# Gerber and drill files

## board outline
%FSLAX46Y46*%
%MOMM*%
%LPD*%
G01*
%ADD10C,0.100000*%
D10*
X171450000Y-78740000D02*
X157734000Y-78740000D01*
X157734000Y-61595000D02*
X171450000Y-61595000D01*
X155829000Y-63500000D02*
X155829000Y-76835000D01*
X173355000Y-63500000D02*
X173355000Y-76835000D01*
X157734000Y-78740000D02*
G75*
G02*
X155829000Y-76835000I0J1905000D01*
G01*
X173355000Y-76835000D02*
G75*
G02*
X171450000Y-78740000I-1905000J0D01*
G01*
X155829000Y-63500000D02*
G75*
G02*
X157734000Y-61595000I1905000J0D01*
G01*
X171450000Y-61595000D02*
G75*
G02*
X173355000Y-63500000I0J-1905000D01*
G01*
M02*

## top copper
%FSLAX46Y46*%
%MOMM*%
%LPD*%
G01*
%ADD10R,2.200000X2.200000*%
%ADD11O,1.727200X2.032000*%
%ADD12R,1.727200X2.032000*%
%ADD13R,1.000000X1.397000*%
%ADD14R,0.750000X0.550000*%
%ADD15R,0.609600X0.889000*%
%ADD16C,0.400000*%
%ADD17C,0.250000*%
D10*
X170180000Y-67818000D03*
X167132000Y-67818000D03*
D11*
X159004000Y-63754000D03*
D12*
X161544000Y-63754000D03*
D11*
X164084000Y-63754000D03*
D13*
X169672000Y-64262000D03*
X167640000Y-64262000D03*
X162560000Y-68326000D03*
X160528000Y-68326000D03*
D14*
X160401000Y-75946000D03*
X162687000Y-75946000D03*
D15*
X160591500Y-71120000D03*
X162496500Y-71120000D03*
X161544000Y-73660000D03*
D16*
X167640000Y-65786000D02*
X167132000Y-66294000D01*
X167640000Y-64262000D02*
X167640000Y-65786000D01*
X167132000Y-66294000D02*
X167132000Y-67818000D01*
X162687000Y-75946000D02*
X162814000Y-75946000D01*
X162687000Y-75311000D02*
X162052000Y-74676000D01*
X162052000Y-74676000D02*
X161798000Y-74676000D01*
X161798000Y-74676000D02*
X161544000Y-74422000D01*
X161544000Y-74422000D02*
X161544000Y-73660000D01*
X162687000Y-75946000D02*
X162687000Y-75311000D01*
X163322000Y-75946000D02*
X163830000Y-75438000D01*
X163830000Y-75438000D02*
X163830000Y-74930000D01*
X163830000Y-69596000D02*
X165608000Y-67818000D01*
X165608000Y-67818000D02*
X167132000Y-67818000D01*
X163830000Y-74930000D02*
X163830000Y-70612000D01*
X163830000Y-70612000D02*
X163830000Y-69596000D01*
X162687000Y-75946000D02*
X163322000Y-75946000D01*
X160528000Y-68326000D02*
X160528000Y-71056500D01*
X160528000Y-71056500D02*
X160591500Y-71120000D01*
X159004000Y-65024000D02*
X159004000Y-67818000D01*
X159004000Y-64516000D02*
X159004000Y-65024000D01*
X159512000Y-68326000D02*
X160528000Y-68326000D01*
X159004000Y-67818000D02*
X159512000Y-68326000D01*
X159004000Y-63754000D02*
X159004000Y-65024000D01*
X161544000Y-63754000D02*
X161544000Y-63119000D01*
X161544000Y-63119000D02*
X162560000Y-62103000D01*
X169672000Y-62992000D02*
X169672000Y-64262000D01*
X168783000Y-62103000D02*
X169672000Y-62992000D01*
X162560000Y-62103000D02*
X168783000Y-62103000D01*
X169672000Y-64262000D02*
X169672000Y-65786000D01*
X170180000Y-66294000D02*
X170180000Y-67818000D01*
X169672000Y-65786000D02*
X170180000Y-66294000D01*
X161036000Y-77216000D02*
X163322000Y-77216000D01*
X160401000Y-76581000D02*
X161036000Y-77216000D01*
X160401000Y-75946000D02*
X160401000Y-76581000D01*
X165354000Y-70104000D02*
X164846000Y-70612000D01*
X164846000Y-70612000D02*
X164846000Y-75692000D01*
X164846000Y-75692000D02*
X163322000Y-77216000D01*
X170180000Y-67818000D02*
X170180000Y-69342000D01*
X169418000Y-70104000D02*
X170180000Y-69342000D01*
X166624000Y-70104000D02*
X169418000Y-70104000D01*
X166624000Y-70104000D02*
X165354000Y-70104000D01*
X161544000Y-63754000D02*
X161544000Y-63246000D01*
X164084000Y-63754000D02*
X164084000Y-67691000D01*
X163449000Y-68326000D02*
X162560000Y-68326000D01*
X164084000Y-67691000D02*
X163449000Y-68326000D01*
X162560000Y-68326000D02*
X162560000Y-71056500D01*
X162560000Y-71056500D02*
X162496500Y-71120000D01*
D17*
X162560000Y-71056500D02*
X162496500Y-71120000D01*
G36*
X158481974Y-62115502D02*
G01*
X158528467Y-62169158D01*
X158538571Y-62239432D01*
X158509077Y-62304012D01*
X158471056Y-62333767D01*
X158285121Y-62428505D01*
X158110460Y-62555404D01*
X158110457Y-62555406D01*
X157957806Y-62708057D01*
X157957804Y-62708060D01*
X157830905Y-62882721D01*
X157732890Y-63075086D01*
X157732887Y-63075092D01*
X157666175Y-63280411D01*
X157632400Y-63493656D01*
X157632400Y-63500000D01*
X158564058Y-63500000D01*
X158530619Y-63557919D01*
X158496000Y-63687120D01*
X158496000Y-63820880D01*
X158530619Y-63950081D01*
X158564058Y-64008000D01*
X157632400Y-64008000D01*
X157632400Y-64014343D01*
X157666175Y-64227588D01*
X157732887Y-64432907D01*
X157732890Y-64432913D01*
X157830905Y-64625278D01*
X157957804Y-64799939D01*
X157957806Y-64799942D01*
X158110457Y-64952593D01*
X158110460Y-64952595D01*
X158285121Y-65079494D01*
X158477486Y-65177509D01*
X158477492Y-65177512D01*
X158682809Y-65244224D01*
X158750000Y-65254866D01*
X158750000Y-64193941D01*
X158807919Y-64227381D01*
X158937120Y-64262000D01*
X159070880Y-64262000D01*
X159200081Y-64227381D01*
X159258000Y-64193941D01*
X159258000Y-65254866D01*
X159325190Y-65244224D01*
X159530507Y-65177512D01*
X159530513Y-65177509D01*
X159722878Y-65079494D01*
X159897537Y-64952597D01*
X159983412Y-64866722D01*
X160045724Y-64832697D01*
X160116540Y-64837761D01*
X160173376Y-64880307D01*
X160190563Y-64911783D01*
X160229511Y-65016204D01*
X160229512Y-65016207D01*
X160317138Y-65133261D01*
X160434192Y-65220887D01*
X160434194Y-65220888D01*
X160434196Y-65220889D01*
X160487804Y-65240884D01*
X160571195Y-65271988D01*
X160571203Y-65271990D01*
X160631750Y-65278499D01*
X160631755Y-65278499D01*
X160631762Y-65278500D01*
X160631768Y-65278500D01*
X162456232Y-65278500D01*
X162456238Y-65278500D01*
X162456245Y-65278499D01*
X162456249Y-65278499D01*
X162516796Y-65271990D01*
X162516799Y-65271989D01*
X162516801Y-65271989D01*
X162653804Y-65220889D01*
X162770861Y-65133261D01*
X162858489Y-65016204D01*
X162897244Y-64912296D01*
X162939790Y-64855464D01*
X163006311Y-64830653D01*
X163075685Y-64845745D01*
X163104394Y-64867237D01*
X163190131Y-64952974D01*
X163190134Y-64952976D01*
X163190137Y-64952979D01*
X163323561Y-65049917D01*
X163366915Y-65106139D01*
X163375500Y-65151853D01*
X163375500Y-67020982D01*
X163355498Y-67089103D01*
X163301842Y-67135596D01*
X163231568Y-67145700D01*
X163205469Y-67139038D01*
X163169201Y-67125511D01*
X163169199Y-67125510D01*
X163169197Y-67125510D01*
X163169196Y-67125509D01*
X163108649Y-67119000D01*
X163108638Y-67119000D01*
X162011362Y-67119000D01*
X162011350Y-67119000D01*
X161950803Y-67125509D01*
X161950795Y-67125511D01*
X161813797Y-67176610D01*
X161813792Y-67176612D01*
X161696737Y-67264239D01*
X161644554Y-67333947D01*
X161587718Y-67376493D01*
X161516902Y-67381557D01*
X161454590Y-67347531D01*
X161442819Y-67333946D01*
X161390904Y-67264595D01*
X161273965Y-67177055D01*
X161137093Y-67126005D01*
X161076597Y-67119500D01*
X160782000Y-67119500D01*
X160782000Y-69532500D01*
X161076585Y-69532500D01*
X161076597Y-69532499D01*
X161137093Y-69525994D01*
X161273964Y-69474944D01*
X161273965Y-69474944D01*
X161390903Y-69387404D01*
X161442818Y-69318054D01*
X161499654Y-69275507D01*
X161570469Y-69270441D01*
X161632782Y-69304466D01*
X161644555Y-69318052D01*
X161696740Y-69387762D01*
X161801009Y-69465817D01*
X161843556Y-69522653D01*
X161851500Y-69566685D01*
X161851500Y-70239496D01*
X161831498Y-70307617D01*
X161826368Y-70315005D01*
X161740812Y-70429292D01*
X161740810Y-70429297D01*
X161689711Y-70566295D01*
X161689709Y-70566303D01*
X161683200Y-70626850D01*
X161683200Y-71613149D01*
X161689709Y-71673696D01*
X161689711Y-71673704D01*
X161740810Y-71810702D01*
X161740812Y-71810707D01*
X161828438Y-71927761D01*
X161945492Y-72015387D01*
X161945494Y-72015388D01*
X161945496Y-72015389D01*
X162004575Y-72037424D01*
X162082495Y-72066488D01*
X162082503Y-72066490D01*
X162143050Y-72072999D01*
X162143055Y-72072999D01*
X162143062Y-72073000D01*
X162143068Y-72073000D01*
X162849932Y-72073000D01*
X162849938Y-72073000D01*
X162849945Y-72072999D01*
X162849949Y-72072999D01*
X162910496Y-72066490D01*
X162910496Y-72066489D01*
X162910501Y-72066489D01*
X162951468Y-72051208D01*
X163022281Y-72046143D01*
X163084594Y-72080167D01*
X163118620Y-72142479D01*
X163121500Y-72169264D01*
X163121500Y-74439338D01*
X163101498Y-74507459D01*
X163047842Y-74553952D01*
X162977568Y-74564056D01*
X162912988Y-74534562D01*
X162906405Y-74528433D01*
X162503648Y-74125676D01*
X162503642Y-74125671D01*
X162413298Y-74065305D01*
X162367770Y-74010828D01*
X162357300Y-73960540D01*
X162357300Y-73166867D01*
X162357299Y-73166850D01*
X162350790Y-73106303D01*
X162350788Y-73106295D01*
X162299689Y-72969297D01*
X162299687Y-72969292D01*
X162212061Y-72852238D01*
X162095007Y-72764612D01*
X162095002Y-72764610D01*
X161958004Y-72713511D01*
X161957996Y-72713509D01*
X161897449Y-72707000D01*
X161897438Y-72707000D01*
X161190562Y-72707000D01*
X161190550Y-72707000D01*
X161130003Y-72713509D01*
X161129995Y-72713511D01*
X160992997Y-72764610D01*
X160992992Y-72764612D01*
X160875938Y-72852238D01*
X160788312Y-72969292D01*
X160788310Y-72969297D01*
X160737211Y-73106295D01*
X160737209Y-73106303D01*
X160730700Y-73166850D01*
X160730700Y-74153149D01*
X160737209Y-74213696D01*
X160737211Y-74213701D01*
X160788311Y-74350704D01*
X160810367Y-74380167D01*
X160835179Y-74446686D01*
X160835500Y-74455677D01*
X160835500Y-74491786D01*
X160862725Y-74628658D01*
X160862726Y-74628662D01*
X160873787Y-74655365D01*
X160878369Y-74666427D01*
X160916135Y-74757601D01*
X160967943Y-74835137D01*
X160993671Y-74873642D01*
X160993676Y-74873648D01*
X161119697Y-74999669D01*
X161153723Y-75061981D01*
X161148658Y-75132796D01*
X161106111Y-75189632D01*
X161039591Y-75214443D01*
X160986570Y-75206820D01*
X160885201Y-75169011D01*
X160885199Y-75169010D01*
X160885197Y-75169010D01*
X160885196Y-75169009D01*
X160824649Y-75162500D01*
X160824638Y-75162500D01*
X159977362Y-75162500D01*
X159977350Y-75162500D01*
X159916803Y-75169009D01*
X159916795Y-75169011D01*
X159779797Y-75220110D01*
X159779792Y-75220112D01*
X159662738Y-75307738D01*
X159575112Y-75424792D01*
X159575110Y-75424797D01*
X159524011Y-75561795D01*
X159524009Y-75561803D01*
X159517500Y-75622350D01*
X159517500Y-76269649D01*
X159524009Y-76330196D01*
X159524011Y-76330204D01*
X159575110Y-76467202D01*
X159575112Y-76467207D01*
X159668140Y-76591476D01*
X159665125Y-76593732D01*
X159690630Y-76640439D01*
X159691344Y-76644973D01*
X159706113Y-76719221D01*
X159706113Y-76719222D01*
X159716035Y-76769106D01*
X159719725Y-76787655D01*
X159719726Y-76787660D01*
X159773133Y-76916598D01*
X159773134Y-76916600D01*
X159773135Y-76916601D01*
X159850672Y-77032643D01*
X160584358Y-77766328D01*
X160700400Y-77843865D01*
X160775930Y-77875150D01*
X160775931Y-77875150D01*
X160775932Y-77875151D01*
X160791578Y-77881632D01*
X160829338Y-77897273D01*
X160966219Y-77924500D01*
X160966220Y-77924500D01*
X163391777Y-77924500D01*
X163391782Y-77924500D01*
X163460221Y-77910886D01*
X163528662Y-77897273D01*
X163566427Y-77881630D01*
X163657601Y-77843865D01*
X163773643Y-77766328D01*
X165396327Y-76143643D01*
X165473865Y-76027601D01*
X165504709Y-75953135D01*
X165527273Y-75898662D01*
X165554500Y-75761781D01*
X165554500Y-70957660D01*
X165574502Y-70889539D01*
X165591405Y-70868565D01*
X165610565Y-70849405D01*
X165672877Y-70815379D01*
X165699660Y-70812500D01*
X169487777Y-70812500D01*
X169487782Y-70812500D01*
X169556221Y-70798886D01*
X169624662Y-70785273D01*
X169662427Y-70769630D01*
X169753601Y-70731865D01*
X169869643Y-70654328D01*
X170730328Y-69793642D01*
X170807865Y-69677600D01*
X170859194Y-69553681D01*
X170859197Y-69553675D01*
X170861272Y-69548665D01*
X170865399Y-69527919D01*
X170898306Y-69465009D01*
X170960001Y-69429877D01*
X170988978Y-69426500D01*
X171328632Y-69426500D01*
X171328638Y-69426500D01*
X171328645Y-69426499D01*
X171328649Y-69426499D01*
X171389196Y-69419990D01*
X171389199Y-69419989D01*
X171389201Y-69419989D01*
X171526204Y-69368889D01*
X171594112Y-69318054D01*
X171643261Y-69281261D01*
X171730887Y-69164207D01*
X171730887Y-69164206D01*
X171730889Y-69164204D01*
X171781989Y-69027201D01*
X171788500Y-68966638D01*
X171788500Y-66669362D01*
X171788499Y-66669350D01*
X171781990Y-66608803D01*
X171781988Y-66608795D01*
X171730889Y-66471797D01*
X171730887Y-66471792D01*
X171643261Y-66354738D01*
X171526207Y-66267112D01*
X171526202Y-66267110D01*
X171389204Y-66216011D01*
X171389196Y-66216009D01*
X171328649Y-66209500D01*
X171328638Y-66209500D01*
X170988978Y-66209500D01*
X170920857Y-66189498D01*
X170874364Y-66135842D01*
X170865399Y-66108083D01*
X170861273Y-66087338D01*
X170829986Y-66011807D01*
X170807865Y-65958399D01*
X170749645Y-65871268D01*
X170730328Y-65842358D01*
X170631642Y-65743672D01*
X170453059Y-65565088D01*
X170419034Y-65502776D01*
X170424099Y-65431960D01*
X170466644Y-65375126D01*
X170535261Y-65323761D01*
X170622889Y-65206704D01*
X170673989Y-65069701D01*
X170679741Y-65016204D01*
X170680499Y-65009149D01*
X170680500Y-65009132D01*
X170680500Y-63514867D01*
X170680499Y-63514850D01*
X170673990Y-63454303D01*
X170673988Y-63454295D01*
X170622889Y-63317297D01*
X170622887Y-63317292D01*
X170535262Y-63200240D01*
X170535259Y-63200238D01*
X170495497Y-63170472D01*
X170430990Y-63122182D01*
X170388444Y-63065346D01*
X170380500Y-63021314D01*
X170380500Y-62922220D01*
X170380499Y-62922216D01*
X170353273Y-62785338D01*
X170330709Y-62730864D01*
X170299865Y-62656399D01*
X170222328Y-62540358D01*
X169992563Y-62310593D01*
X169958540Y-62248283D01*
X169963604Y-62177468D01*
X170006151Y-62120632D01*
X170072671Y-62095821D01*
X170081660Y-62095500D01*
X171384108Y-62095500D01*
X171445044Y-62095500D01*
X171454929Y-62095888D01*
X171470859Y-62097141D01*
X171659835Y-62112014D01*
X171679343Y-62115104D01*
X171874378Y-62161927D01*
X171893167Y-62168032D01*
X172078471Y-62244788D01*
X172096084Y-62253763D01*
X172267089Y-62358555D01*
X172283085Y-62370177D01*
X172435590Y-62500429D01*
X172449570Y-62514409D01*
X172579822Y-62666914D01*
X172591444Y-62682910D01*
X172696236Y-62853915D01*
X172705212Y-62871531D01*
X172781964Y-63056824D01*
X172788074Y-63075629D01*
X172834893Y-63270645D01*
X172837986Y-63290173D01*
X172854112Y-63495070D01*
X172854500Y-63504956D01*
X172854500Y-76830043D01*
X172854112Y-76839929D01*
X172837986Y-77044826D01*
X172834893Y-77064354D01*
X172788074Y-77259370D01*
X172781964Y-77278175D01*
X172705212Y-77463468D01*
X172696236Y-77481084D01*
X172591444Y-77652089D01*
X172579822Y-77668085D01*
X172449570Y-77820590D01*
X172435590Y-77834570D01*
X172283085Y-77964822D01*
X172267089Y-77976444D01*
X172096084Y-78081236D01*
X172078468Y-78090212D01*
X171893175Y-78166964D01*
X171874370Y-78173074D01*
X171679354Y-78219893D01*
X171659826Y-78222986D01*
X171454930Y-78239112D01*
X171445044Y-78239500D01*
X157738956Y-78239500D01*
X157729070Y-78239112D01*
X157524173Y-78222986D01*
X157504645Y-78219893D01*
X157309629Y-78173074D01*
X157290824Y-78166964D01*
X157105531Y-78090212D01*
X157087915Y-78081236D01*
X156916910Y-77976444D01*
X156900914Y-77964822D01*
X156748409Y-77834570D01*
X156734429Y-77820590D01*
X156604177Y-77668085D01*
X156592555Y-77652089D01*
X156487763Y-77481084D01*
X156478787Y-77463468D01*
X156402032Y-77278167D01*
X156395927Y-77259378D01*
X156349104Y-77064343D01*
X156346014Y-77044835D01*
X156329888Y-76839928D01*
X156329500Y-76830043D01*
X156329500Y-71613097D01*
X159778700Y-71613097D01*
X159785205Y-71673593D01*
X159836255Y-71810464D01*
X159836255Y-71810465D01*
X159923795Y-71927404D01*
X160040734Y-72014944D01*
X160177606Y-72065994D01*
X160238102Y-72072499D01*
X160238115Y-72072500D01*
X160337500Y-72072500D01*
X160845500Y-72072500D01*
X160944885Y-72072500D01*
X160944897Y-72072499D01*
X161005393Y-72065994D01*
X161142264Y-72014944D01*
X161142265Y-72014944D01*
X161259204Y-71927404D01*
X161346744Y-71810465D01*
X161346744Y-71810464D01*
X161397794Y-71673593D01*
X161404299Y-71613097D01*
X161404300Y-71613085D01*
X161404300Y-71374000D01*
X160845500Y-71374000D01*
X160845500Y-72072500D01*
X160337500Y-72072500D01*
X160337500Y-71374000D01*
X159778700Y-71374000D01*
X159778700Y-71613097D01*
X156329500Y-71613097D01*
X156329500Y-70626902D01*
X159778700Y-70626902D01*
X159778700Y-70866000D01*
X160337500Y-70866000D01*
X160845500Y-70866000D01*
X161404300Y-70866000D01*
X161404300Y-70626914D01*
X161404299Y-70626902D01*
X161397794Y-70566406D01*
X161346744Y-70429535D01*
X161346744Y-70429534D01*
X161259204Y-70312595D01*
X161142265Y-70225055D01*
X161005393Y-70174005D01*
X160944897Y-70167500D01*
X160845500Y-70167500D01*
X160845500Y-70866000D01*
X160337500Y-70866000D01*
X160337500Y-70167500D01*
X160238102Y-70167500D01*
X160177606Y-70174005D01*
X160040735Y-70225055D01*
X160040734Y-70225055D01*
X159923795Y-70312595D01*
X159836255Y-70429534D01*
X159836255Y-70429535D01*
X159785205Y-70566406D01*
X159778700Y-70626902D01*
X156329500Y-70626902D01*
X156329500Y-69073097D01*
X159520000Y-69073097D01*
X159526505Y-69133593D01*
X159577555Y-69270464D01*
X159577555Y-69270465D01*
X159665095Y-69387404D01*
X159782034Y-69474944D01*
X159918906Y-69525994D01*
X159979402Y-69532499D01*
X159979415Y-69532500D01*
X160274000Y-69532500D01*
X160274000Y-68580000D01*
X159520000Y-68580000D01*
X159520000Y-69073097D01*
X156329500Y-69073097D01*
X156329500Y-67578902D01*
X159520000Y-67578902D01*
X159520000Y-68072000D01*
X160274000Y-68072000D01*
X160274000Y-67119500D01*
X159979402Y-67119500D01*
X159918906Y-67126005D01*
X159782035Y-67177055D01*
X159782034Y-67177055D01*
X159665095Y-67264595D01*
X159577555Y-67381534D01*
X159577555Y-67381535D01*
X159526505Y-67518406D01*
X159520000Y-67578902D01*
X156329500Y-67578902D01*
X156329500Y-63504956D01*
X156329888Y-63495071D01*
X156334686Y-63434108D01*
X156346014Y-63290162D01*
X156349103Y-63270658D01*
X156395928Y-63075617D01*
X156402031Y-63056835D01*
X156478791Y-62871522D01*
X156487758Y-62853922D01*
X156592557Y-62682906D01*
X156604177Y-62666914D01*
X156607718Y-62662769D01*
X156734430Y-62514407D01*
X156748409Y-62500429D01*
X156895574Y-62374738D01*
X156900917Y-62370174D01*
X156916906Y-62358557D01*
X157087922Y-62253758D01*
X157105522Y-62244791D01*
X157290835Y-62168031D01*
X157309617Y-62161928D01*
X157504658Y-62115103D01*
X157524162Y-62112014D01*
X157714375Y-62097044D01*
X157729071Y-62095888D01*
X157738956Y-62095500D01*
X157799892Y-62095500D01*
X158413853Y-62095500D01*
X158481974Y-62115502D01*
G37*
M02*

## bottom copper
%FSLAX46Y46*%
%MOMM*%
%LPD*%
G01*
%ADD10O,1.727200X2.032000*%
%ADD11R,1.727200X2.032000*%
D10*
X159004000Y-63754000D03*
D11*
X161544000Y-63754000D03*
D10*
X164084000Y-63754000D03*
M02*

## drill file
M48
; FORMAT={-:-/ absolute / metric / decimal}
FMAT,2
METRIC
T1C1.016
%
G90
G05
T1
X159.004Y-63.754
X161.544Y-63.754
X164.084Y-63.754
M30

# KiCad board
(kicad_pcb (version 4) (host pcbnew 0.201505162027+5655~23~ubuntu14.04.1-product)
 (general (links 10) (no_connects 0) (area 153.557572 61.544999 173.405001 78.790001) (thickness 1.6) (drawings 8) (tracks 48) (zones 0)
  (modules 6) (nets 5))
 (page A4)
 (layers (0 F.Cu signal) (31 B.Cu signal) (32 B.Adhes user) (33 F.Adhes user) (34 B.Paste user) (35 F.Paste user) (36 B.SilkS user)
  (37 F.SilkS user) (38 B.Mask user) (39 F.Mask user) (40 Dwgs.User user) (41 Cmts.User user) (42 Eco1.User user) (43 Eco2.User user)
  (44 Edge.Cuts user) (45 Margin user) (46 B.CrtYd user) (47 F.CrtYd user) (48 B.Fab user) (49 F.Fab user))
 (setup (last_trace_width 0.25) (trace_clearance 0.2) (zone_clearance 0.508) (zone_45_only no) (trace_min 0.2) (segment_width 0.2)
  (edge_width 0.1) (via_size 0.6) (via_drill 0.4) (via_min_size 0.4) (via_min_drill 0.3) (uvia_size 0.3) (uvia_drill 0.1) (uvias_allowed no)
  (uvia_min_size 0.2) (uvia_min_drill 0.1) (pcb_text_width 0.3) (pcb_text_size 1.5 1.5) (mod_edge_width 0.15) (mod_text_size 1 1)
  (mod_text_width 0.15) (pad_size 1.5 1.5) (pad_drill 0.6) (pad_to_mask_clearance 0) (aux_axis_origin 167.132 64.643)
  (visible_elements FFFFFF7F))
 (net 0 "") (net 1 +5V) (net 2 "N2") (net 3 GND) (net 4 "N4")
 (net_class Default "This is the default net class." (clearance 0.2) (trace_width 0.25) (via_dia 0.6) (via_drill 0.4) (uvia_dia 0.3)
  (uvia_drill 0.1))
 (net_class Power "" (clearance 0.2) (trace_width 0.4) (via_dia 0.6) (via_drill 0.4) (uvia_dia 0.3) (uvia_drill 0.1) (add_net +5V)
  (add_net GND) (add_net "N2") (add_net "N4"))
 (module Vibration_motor (layer F.Cu) (at 168.656 67.818 180)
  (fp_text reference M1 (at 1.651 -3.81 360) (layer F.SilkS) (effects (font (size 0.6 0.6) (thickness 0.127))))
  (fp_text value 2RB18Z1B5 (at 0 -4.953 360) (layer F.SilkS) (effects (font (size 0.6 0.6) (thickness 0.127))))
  (pad 1 smd rect (at -1.524 0 180) (size 2.2 2.2) (layers F.Cu F.Paste F.Mask) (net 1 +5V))
  (pad 2 smd rect (at 1.524 0 180) (size 2.2 2.2) (layers F.Cu F.Paste F.Mask) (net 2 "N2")))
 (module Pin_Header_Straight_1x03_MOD (layer F.Cu) (at 159.004 63.754 90)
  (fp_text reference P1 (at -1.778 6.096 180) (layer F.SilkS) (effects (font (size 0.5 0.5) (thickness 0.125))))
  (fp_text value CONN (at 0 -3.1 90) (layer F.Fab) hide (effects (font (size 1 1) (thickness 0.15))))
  (pad 1 thru_hole oval (at 0 0 90) (size 2.032 1.7272) (drill 1.016) (layers *.Cu *.Mask F.SilkS) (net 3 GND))
  (pad 2 thru_hole rect (at 0 2.54 90) (size 2.032 1.7272) (drill 1.016) (layers *.Cu *.Mask F.SilkS) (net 1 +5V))
  (pad 3 thru_hole oval (at 0 5.08 90) (size 2.032 1.7272) (drill 1.016) (layers *.Cu *.Mask F.SilkS) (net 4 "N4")))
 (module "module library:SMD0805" (layer F.Cu) (at 168.656 64.262 180)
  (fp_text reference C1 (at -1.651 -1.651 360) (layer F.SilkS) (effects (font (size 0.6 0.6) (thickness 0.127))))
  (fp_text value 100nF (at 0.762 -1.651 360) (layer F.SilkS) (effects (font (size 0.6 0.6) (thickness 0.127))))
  (pad 1 smd rect (at -1.016 0 180) (size 1 1.397) (layers F.Cu F.Paste F.Mask) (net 1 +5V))
  (pad 2 smd rect (at 1.016 0 180) (size 1 1.397) (layers F.Cu F.Paste F.Mask) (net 2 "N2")))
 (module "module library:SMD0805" (layer F.Cu) (at 161.544 68.326 180)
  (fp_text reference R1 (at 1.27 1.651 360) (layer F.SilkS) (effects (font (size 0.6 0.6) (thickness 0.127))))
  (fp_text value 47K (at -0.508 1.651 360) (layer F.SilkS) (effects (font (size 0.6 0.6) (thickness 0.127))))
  (pad 1 smd rect (at -1.016 0 180) (size 1 1.397) (layers F.Cu F.Paste F.Mask) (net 4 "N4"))
  (pad 2 smd rect (at 1.016 0 180) (size 1 1.397) (layers F.Cu F.Paste F.Mask) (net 3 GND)))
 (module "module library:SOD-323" (layer F.Cu) (at 161.544 75.946)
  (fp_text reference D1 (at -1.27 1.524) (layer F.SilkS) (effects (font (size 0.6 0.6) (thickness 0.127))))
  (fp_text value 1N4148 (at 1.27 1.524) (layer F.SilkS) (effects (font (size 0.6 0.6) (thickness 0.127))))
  (pad 1 smd rect (at -1.143 0) (size 0.75 0.55) (layers F.Cu F.Paste F.Mask) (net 1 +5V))
  (pad 2 smd rect (at 1.143 0) (size 0.75 0.55) (layers F.Cu F.Paste F.Mask) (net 2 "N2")))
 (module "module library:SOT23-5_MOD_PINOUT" (layer F.Cu) (at 161.544 72.39 180)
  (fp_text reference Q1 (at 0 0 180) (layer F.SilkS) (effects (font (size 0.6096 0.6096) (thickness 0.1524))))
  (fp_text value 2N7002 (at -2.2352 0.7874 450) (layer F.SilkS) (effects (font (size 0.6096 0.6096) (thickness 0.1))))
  (pad 3 smd rect (at 0.9525 1.27 180) (size 0.6096 0.889) (layers F.Cu F.Paste F.Mask) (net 3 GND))
  (pad 2 smd rect (at -0.9525 1.27 180) (size 0.6096 0.889) (layers F.Cu F.Paste F.Mask) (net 4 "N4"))
  (pad 1 smd rect (at 0 -1.27 180) (size 0.6096 0.889) (layers F.Cu F.Paste F.Mask) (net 2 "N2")))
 (gr_line (start 171.45 78.74) (end 157.734 78.74) (angle 90) (layer Edge.Cuts) (width 0.1))
 (gr_line (start 157.734 61.595) (end 171.45 61.595) (angle 90) (layer Edge.Cuts) (width 0.1))
 (gr_line (start 155.829 63.5) (end 155.829 76.835) (angle 90) (layer Edge.Cuts) (width 0.1))
 (gr_line (start 173.355 63.5) (end 173.355 76.835) (angle 90) (layer Edge.Cuts) (width 0.1))
 (gr_arc (start 157.734 76.835) (end 157.734 78.74) (angle 90) (layer Edge.Cuts) (width 0.1))
 (gr_arc (start 171.45 76.835) (end 173.355 76.835) (angle 90) (layer Edge.Cuts) (width 0.1))
 (gr_arc (start 157.734 63.5) (end 155.829 63.5) (angle 90) (layer Edge.Cuts) (width 0.1))
 (gr_arc (start 171.45 63.5) (end 171.45 61.595) (angle 90) (layer Edge.Cuts) (width 0.1))
 (segment (start 167.64 65.786) (end 167.132 66.294) (width 0.4) (layer F.Cu) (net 2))
 (segment (start 167.64 64.262) (end 167.64 65.786) (width 0.4) (layer F.Cu) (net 2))
 (segment (start 167.132 66.294) (end 167.132 67.818) (width 0.4) (layer F.Cu) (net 2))
 (segment (start 162.687 75.946) (end 162.814 75.946) (width 0.4) (layer F.Cu) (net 2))
 (segment (start 162.687 75.311) (end 162.052 74.676) (width 0.4) (layer F.Cu) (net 2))
 (segment (start 162.052 74.676) (end 161.798 74.676) (width 0.4) (layer F.Cu) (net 2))
 (segment (start 161.798 74.676) (end 161.544 74.422) (width 0.4) (layer F.Cu) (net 2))
 (segment (start 161.544 74.422) (end 161.544 73.66) (width 0.4) (layer F.Cu) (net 2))
 (segment (start 162.687 75.946) (end 162.687 75.311) (width 0.4) (layer F.Cu) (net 2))
 (segment (start 163.322 75.946) (end 163.83 75.438) (width 0.4) (layer F.Cu) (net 2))
 (segment (start 163.83 75.438) (end 163.83 74.93) (width 0.4) (layer F.Cu) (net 2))
 (segment (start 163.83 69.596) (end 165.608 67.818) (width 0.4) (layer F.Cu) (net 2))
 (segment (start 165.608 67.818) (end 167.132 67.818) (width 0.4) (layer F.Cu) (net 2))
 (segment (start 163.83 74.93) (end 163.83 70.612) (width 0.4) (layer F.Cu) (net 2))
 (segment (start 163.83 70.612) (end 163.83 69.596) (width 0.4) (layer F.Cu) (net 2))
 (segment (start 162.687 75.946) (end 163.322 75.946) (width 0.4) (layer F.Cu) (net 2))
 (segment (start 160.528 68.326) (end 160.528 71.0565) (width 0.4) (layer F.Cu) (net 3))
 (segment (start 160.528 71.0565) (end 160.5915 71.12) (width 0.4) (layer F.Cu) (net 3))
 (segment (start 159.004 65.024) (end 159.004 67.818) (width 0.4) (layer F.Cu) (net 3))
 (segment (start 159.004 64.516) (end 159.004 65.024) (width 0.4) (layer F.Cu) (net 3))
 (segment (start 159.512 68.326) (end 160.528 68.326) (width 0.4) (layer F.Cu) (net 3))
 (segment (start 159.004 67.818) (end 159.512 68.326) (width 0.4) (layer F.Cu) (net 3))
 (segment (start 159.004 63.754) (end 159.004 65.024) (width 0.4) (layer F.Cu) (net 3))
 (segment (start 161.544 63.754) (end 161.544 63.119) (width 0.4) (layer F.Cu) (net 1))
 (segment (start 161.544 63.119) (end 162.56 62.103) (width 0.4) (layer F.Cu) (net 1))
 (segment (start 169.672 62.992) (end 169.672 64.262) (width 0.4) (layer F.Cu) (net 1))
 (segment (start 168.783 62.103) (end 169.672 62.992) (width 0.4) (layer F.Cu) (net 1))
 (segment (start 162.56 62.103) (end 168.783 62.103) (width 0.4) (layer F.Cu) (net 1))
 (segment (start 169.672 64.262) (end 169.672 65.786) (width 0.4) (layer F.Cu) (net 1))
 (segment (start 170.18 66.294) (end 170.18 67.818) (width 0.4) (layer F.Cu) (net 1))
 (segment (start 169.672 65.786) (end 170.18 66.294) (width 0.4) (layer F.Cu) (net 1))
 (segment (start 161.036 77.216) (end 163.322 77.216) (width 0.4) (layer F.Cu) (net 1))
 (segment (start 160.401 76.581) (end 161.036 77.216) (width 0.4) (layer F.Cu) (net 1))
 (segment (start 160.401 75.946) (end 160.401 76.581) (width 0.4) (layer F.Cu) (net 1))
 (segment (start 165.354 70.104) (end 164.846 70.612) (width 0.4) (layer F.Cu) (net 1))
 (segment (start 164.846 70.612) (end 164.846 75.692) (width 0.4) (layer F.Cu) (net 1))
 (segment (start 164.846 75.692) (end 163.322 77.216) (width 0.4) (layer F.Cu) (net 1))
 (segment (start 170.18 67.818) (end 170.18 69.342) (width 0.4) (layer F.Cu) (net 1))
 (segment (start 169.418 70.104) (end 170.18 69.342) (width 0.4) (layer F.Cu) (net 1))
 (segment (start 166.624 70.104) (end 169.418 70.104) (width 0.4) (layer F.Cu) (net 1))
 (segment (start 166.624 70.104) (end 165.354 70.104) (width 0.4) (layer F.Cu) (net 1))
 (segment (start 161.544 63.754) (end 161.544 63.246) (width 0.4) (layer F.Cu) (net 1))
 (segment (start 164.084 63.754) (end 164.084 67.691) (width 0.4) (layer F.Cu) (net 4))
 (segment (start 163.449 68.326) (end 162.56 68.326) (width 0.4) (layer F.Cu) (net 4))
 (segment (start 164.084 67.691) (end 163.449 68.326) (width 0.4) (layer F.Cu) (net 4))
 (segment (start 162.56 68.326) (end 162.56 71.0565) (width 0.4) (layer F.Cu) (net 4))
 (segment (start 162.56 71.0565) (end 162.4965 71.12) (width 0.4) (layer F.Cu) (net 4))
 (segment (start 162.56 71.0565) (end 162.4965 71.12) (width 0.25) (layer F.Cu) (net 4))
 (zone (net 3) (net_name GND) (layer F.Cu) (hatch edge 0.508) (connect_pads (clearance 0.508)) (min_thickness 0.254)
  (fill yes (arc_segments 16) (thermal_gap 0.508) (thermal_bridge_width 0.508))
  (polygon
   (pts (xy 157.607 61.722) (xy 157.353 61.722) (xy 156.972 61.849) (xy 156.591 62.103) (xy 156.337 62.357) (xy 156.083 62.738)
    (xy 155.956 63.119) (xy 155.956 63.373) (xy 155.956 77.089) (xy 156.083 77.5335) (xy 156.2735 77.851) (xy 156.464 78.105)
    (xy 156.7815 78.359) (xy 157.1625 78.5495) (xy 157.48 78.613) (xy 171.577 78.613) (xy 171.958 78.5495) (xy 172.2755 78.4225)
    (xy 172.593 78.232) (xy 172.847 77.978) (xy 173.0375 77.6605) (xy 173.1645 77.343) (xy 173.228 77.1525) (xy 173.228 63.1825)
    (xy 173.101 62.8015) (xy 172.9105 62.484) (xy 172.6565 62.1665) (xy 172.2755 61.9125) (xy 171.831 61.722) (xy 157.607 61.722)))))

